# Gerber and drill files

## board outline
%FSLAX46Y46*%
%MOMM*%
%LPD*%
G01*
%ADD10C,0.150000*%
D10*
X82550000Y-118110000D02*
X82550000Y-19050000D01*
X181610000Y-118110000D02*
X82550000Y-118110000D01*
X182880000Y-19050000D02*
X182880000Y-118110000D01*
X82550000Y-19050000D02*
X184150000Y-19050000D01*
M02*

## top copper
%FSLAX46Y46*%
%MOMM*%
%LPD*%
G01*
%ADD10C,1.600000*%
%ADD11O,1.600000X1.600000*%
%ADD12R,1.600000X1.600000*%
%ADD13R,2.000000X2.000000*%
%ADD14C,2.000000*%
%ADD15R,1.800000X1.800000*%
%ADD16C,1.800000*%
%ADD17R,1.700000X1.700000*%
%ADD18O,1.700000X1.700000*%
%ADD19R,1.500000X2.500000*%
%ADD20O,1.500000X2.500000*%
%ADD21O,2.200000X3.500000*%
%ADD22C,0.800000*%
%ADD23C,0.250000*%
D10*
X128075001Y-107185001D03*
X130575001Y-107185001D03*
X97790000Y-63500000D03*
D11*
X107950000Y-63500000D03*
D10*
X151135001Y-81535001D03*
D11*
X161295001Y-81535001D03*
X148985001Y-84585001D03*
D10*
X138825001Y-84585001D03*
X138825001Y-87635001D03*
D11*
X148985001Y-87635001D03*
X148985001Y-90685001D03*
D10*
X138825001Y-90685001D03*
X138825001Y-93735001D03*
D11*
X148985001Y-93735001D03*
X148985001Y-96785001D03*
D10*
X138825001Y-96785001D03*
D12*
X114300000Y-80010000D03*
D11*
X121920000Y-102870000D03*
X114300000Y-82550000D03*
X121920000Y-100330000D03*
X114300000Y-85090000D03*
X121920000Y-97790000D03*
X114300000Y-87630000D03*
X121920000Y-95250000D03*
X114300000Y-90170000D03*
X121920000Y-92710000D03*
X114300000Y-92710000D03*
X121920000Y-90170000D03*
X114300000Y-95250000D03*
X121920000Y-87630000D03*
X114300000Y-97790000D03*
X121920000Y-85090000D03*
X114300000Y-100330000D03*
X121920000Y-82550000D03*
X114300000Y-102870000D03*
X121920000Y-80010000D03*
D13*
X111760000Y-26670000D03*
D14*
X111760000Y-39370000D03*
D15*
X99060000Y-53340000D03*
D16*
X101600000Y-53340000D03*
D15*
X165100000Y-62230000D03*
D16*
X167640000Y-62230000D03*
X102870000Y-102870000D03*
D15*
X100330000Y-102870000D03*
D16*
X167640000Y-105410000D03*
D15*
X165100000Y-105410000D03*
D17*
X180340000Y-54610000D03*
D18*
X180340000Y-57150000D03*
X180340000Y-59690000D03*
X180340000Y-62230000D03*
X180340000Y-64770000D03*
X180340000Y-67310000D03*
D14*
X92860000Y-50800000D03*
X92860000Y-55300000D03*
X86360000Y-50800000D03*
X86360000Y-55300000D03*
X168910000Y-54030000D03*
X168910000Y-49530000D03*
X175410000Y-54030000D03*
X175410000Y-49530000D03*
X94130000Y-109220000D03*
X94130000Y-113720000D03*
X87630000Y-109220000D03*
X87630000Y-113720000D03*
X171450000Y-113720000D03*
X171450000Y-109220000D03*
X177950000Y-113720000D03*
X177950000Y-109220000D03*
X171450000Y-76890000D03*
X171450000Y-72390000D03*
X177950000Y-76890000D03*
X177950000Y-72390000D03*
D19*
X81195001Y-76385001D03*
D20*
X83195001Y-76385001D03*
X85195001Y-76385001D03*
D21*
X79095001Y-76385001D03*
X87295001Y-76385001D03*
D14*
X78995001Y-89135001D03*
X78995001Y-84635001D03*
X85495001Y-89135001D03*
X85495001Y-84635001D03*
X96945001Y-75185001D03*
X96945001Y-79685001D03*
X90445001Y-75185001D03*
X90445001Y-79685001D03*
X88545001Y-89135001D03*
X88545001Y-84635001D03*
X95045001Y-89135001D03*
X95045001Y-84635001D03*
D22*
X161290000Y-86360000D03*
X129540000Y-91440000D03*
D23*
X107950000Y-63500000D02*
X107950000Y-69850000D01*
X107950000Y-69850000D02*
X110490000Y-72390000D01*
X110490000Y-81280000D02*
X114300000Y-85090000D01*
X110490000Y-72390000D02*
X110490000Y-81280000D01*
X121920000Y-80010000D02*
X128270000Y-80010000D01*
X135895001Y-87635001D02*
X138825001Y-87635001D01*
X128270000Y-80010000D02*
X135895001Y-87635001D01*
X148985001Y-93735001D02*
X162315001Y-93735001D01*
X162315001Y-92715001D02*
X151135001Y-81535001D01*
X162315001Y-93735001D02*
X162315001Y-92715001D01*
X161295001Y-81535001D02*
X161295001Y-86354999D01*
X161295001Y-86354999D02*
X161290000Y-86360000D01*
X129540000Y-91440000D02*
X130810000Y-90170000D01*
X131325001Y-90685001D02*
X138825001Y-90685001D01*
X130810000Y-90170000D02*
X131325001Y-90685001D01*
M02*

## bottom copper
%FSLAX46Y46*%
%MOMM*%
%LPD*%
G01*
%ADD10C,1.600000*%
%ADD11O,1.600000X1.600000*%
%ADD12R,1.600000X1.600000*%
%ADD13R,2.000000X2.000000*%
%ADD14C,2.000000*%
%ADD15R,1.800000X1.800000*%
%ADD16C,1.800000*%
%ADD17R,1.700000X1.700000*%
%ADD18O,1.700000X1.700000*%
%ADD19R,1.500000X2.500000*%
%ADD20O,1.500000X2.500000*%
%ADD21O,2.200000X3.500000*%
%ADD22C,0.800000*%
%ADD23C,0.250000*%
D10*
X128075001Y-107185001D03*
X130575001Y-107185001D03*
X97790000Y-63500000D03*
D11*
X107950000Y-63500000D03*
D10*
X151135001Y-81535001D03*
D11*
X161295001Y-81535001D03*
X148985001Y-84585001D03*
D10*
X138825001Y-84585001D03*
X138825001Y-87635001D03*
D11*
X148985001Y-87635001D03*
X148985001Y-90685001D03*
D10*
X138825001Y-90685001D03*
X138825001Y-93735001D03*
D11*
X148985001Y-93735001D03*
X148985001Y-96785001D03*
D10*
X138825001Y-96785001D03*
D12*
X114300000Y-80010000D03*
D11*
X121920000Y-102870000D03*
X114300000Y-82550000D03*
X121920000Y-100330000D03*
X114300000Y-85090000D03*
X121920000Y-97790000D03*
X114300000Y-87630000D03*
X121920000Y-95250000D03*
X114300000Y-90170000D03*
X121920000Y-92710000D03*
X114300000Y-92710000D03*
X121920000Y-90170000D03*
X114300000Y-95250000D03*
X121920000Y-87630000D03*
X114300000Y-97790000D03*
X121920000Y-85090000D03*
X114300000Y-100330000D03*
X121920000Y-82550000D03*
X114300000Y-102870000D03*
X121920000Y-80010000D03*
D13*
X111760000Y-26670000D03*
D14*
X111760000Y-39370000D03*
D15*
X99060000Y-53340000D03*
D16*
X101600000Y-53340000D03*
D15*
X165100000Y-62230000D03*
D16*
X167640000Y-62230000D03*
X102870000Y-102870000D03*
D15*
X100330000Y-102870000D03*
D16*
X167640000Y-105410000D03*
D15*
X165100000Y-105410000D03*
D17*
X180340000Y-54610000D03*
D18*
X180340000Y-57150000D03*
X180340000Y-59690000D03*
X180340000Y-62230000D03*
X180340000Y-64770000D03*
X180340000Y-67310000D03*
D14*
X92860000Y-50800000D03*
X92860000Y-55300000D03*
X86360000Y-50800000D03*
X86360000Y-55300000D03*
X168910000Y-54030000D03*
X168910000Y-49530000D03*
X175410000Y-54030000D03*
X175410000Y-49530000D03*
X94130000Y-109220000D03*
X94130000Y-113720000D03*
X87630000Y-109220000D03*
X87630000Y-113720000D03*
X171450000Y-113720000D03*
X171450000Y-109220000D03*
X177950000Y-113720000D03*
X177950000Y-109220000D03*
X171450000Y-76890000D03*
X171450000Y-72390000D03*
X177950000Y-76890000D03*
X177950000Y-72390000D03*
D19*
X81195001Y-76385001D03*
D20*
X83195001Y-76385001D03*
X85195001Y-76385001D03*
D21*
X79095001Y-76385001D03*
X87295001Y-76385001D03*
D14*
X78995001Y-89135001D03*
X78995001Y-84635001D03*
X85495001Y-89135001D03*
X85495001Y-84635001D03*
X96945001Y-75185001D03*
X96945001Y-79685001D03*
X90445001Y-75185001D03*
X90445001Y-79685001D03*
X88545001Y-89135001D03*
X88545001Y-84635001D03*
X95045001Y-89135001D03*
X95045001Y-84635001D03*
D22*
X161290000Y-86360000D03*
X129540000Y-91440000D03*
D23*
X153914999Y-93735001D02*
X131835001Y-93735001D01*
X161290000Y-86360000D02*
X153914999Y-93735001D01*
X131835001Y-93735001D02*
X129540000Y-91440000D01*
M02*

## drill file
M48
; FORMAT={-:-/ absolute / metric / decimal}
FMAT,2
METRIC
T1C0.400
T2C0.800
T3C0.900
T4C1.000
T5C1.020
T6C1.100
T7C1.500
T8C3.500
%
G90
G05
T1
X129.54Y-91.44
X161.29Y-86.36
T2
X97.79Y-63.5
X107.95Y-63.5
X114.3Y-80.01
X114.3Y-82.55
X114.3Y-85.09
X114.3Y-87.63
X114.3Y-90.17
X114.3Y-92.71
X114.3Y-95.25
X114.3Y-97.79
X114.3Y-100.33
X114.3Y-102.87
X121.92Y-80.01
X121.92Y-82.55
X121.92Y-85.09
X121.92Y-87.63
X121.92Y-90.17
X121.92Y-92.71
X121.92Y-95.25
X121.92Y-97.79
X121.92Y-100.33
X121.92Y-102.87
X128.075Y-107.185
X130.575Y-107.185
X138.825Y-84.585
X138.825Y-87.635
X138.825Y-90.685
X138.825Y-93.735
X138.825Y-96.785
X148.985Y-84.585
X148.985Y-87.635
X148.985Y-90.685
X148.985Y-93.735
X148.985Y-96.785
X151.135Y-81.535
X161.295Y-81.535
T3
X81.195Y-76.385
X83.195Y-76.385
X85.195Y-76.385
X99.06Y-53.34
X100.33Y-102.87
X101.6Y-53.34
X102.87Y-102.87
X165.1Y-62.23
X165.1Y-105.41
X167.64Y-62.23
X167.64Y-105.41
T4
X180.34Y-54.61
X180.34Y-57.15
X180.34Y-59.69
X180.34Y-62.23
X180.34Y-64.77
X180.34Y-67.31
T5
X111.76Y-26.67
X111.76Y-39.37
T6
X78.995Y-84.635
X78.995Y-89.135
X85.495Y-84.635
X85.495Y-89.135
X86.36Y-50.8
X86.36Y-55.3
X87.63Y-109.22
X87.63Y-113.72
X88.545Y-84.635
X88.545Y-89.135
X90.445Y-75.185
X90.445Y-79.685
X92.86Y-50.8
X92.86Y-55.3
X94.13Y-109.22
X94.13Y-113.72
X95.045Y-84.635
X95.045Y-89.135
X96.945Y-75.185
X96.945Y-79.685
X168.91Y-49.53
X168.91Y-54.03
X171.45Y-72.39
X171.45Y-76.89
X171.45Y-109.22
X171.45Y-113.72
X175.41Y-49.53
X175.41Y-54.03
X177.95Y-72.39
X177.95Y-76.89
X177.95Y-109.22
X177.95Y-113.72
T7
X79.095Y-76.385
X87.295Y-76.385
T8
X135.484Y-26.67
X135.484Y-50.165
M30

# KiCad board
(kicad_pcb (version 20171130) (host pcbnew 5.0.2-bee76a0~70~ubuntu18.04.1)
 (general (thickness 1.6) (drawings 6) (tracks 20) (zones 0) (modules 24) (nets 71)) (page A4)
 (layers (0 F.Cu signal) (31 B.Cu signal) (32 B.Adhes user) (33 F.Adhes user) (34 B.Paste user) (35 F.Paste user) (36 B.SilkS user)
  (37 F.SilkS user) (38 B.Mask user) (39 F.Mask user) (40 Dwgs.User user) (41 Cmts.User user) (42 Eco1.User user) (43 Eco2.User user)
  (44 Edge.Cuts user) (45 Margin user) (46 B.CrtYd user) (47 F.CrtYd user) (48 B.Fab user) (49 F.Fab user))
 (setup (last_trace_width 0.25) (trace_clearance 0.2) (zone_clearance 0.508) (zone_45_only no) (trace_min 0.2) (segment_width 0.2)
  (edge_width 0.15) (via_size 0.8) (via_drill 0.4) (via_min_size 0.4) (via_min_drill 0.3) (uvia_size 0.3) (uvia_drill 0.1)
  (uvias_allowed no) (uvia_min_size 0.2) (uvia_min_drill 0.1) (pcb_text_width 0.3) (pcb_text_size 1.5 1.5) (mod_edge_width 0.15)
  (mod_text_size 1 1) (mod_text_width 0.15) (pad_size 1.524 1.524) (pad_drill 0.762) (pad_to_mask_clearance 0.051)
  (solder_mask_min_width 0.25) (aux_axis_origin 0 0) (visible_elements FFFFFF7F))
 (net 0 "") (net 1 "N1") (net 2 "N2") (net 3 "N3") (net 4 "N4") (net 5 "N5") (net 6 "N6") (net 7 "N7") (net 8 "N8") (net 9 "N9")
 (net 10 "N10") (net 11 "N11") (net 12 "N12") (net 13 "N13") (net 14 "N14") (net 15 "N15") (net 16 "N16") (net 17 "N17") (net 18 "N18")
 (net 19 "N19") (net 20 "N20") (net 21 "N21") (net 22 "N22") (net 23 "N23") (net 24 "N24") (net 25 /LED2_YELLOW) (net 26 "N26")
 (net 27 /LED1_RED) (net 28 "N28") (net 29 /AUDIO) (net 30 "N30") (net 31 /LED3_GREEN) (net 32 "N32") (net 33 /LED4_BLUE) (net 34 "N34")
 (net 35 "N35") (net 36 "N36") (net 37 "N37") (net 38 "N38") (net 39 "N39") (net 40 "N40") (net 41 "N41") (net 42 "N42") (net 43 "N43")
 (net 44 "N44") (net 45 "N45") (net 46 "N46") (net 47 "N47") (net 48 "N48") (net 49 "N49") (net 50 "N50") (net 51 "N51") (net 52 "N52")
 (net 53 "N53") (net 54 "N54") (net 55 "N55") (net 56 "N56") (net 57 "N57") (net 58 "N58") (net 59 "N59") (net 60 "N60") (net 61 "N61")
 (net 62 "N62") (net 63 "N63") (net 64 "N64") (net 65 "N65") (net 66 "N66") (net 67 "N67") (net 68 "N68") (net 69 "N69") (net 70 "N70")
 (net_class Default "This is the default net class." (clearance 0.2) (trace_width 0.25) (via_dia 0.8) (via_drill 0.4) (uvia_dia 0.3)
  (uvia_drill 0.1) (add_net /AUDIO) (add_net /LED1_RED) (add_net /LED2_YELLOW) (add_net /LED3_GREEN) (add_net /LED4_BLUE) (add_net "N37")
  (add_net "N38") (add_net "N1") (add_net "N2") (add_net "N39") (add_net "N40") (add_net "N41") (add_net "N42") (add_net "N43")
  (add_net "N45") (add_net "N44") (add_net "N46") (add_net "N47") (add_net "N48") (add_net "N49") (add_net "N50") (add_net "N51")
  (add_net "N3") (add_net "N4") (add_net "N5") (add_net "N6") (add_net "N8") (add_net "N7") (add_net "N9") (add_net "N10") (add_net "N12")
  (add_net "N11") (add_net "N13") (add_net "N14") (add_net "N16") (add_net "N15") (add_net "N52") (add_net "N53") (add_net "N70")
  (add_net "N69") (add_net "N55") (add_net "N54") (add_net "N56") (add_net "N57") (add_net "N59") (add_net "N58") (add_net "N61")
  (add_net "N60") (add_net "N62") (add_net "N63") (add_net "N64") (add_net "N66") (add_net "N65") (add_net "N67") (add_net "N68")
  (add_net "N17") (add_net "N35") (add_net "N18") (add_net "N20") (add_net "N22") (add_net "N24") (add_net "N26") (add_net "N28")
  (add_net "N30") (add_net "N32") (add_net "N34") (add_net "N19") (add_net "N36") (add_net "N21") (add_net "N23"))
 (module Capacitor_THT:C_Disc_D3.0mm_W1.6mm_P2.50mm (layer F.Cu) (at 128.075001 107.185001)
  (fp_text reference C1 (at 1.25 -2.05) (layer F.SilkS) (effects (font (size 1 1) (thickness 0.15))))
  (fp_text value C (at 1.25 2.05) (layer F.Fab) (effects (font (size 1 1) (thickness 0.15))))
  (pad 1 thru_hole circle (at 0 0) (size 1.6 1.6) (drill 0.8) (layers *.Cu *.Mask) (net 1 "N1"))
  (pad 2 thru_hole circle (at 2.5 0) (size 1.6 1.6) (drill 0.8) (layers *.Cu *.Mask) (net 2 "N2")))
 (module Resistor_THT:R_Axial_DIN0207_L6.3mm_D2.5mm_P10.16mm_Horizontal (layer F.Cu) (at 97.79 63.5)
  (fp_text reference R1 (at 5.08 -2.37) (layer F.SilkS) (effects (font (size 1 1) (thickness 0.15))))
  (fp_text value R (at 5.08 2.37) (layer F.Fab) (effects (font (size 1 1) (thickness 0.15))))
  (pad 1 thru_hole circle (at 0 0) (size 1.6 1.6) (drill 0.8) (layers *.Cu *.Mask) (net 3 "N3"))
  (pad 2 thru_hole oval (at 10.16 0) (size 1.6 1.6) (drill 0.8) (layers *.Cu *.Mask) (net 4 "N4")))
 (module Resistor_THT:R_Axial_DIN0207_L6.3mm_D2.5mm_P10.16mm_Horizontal (layer F.Cu) (at 151.135001 81.535001)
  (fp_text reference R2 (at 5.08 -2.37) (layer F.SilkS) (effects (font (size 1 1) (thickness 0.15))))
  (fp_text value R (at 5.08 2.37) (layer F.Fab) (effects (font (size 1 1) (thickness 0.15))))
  (pad 1 thru_hole circle (at 0 0) (size 1.6 1.6) (drill 0.8) (layers *.Cu *.Mask) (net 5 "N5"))
  (pad 2 thru_hole oval (at 10.16 0) (size 1.6 1.6) (drill 0.8) (layers *.Cu *.Mask) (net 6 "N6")))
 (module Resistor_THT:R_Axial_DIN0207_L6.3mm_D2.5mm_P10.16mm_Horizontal (layer F.Cu) (at 138.825001 84.585001)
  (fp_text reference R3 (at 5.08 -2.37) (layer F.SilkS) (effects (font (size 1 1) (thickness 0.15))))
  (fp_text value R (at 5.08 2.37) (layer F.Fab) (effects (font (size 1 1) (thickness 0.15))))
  (pad 2 thru_hole oval (at 10.16 0) (size 1.6 1.6) (drill 0.8) (layers *.Cu *.Mask) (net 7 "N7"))
  (pad 1 thru_hole circle (at 0 0) (size 1.6 1.6) (drill 0.8) (layers *.Cu *.Mask) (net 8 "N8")))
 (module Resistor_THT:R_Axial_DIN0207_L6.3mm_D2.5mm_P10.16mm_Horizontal (layer F.Cu) (at 138.825001 87.635001)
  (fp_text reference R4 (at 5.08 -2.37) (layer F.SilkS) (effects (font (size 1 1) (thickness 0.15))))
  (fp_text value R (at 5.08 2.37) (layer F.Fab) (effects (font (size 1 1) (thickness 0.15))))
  (pad 1 thru_hole circle (at 0 0) (size 1.6 1.6) (drill 0.8) (layers *.Cu *.Mask) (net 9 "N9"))
  (pad 2 thru_hole oval (at 10.16 0) (size 1.6 1.6) (drill 0.8) (layers *.Cu *.Mask) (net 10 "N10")))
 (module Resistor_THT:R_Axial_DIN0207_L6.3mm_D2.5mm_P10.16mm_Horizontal (layer F.Cu) (at 138.825001 90.685001)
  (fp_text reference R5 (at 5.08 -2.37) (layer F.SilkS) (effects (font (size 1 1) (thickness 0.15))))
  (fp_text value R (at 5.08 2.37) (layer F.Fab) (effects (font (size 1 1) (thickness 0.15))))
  (pad 2 thru_hole oval (at 10.16 0) (size 1.6 1.6) (drill 0.8) (layers *.Cu *.Mask) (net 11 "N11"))
  (pad 1 thru_hole circle (at 0 0) (size 1.6 1.6) (drill 0.8) (layers *.Cu *.Mask) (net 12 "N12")))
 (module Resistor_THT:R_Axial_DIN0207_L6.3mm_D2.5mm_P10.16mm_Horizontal (layer F.Cu) (at 138.825001 93.735001)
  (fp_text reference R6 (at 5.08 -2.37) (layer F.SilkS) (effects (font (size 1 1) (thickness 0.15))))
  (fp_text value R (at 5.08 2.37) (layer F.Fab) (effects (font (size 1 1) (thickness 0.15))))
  (pad 1 thru_hole circle (at 0 0) (size 1.6 1.6) (drill 0.8) (layers *.Cu *.Mask) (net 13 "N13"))
  (pad 2 thru_hole oval (at 10.16 0) (size 1.6 1.6) (drill 0.8) (layers *.Cu *.Mask) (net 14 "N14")))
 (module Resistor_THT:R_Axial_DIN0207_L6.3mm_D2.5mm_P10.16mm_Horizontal (layer F.Cu) (at 138.825001 96.785001)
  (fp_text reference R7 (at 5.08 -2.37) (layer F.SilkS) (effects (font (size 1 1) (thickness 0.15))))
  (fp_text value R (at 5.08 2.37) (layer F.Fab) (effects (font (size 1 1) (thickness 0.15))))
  (pad 2 thru_hole oval (at 10.16 0) (size 1.6 1.6) (drill 0.8) (layers *.Cu *.Mask) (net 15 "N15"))
  (pad 1 thru_hole circle (at 0 0) (size 1.6 1.6) (drill 0.8) (layers *.Cu *.Mask) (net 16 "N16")))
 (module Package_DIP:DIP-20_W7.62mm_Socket (layer F.Cu) (at 114.3 80.01)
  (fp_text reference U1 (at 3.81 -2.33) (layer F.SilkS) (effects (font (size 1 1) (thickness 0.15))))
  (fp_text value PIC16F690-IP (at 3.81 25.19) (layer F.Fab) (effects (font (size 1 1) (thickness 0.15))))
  (pad 1 thru_hole rect (at 0 0) (size 1.6 1.6) (drill 0.8) (layers *.Cu *.Mask) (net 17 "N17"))
  (pad 11 thru_hole oval (at 7.62 22.86) (size 1.6 1.6) (drill 0.8) (layers *.Cu *.Mask) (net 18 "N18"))
  (pad 2 thru_hole oval (at 0 2.54) (size 1.6 1.6) (drill 0.8) (layers *.Cu *.Mask) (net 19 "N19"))
  (pad 12 thru_hole oval (at 7.62 20.32) (size 1.6 1.6) (drill 0.8) (layers *.Cu *.Mask) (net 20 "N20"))
  (pad 3 thru_hole oval (at 0 5.08) (size 1.6 1.6) (drill 0.8) (layers *.Cu *.Mask) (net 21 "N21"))
  (pad 13 thru_hole oval (at 7.62 17.78) (size 1.6 1.6) (drill 0.8) (layers *.Cu *.Mask) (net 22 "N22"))
  (pad 4 thru_hole oval (at 0 7.62) (size 1.6 1.6) (drill 0.8) (layers *.Cu *.Mask) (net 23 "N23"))
  (pad 14 thru_hole oval (at 7.62 15.24) (size 1.6 1.6) (drill 0.8) (layers *.Cu *.Mask) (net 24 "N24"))
  (pad 5 thru_hole oval (at 0 10.16) (size 1.6 1.6) (drill 0.8) (layers *.Cu *.Mask) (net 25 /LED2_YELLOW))
  (pad 15 thru_hole oval (at 7.62 12.7) (size 1.6 1.6) (drill 0.8) (layers *.Cu *.Mask) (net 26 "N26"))
  (pad 6 thru_hole oval (at 0 12.7) (size 1.6 1.6) (drill 0.8) (layers *.Cu *.Mask) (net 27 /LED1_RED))
  (pad 16 thru_hole oval (at 7.62 10.16) (size 1.6 1.6) (drill 0.8) (layers *.Cu *.Mask) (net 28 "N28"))
  (pad 7 thru_hole oval (at 0 15.24) (size 1.6 1.6) (drill 0.8) (layers *.Cu *.Mask) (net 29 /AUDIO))
  (pad 17 thru_hole oval (at 7.62 7.62) (size 1.6 1.6) (drill 0.8) (layers *.Cu *.Mask) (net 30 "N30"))
  (pad 8 thru_hole oval (at 0 17.78) (size 1.6 1.6) (drill 0.8) (layers *.Cu *.Mask) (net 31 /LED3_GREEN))
  (pad 18 thru_hole oval (at 7.62 5.08) (size 1.6 1.6) (drill 0.8) (layers *.Cu *.Mask) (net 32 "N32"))
  (pad 9 thru_hole oval (at 0 20.32) (size 1.6 1.6) (drill 0.8) (layers *.Cu *.Mask) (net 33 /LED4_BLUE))
  (pad 19 thru_hole oval (at 7.62 2.54) (size 1.6 1.6) (drill 0.8) (layers *.Cu *.Mask) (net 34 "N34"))
  (pad 10 thru_hole oval (at 0 22.86) (size 1.6 1.6) (drill 0.8) (layers *.Cu *.Mask) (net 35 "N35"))
  (pad 20 thru_hole oval (at 7.62 0) (size 1.6 1.6) (drill 0.8) (layers *.Cu *.Mask) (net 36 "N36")))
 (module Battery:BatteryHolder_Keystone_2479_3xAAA (layer F.Cu) (at 111.76 26.67)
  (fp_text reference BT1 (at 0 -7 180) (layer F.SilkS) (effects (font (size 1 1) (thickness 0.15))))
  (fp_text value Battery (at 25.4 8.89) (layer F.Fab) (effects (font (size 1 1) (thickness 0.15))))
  (pad 1 thru_hole rect (at 0 0) (size 2 2) (drill 1.02) (layers *.Cu *.Mask) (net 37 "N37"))
  (pad 2 thru_hole circle (at 0 12.7) (size 2 2) (drill 1.02) (layers *.Cu *.Mask) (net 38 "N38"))
  (pad "" np_thru_hole circle (at 23.7236 23.495) (size 3.5 3.5) (drill 3.5) (layers *.Cu *.Mask))
  (pad "" np_thru_hole circle (at 23.7236 0) (size 3.5 3.5) (drill 3.5) (layers *.Cu *.Mask)))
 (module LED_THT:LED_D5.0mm (layer F.Cu) (at 99.06 53.34)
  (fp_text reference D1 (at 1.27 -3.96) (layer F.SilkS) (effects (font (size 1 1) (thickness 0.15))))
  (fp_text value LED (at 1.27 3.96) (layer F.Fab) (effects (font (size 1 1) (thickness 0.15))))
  (pad 1 thru_hole rect (at 0 0) (size 1.8 1.8) (drill 0.9) (layers *.Cu *.Mask) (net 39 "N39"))
  (pad 2 thru_hole circle (at 2.54 0) (size 1.8 1.8) (drill 0.9) (layers *.Cu *.Mask) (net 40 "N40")))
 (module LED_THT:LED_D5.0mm (layer F.Cu) (at 165.1 62.23)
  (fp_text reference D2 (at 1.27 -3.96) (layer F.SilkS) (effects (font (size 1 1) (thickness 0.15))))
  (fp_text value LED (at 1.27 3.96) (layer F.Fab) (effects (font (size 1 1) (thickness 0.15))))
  (pad 1 thru_hole rect (at 0 0) (size 1.8 1.8) (drill 0.9) (layers *.Cu *.Mask) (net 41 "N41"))
  (pad 2 thru_hole circle (at 2.54 0) (size 1.8 1.8) (drill 0.9) (layers *.Cu *.Mask) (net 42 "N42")))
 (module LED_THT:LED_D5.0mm (layer F.Cu) (at 100.33 102.87)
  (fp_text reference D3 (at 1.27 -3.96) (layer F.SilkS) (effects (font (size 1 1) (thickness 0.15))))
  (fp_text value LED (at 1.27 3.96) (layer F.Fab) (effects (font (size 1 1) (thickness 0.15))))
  (pad 2 thru_hole circle (at 2.54 0) (size 1.8 1.8) (drill 0.9) (layers *.Cu *.Mask) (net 31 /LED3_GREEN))
  (pad 1 thru_hole rect (at 0 0) (size 1.8 1.8) (drill 0.9) (layers *.Cu *.Mask) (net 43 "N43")))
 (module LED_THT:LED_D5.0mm (layer F.Cu) (at 165.1 105.41)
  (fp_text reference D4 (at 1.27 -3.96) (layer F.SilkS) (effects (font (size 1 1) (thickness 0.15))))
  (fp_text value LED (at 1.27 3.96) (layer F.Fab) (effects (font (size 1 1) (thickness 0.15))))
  (pad 2 thru_hole circle (at 2.54 0) (size 1.8 1.8) (drill 0.9) (layers *.Cu *.Mask) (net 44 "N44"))
  (pad 1 thru_hole rect (at 0 0) (size 1.8 1.8) (drill 0.9) (layers *.Cu *.Mask) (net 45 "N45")))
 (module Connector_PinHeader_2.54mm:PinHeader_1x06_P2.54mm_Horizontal (layer F.Cu) (at 180.34 54.61)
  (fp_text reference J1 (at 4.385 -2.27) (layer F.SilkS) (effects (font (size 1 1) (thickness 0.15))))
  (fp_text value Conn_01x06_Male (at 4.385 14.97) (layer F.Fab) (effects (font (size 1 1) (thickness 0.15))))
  (pad 1 thru_hole rect (at 0 0) (size 1.7 1.7) (drill 1) (layers *.Cu *.Mask) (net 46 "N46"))
  (pad 2 thru_hole oval (at 0 2.54) (size 1.7 1.7) (drill 1) (layers *.Cu *.Mask) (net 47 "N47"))
  (pad 3 thru_hole oval (at 0 5.08) (size 1.7 1.7) (drill 1) (layers *.Cu *.Mask) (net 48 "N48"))
  (pad 4 thru_hole oval (at 0 7.62) (size 1.7 1.7) (drill 1) (layers *.Cu *.Mask) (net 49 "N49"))
  (pad 5 thru_hole oval (at 0 10.16) (size 1.7 1.7) (drill 1) (layers *.Cu *.Mask) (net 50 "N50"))
  (pad 6 thru_hole oval (at 0 12.7) (size 1.7 1.7) (drill 1) (layers *.Cu *.Mask) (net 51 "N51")))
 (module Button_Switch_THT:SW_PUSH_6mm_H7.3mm (layer F.Cu) (at 86.36 50.8)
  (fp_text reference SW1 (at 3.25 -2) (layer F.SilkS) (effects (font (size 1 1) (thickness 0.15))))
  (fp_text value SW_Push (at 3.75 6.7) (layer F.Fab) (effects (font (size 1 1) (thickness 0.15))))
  (pad 1 thru_hole circle (at 6.5 0 90) (size 2 2) (drill 1.1) (layers *.Cu *.Mask) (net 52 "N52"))
  (pad 2 thru_hole circle (at 6.5 4.5 90) (size 2 2) (drill 1.1) (layers *.Cu *.Mask) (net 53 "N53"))
  (pad 1 thru_hole circle (at 0 0 90) (size 2 2) (drill 1.1) (layers *.Cu *.Mask) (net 52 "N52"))
  (pad 2 thru_hole circle (at 0 4.5 90) (size 2 2) (drill 1.1) (layers *.Cu *.Mask) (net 53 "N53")))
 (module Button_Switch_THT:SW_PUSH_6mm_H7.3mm (layer F.Cu) (at 168.91 49.53)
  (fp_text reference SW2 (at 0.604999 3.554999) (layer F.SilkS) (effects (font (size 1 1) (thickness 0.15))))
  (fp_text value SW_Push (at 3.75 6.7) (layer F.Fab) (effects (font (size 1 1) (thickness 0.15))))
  (pad 2 thru_hole circle (at 0 4.5 90) (size 2 2) (drill 1.1) (layers *.Cu *.Mask) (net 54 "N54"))
  (pad 1 thru_hole circle (at 0 0 90) (size 2 2) (drill 1.1) (layers *.Cu *.Mask) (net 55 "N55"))
  (pad 2 thru_hole circle (at 6.5 4.5 90) (size 2 2) (drill 1.1) (layers *.Cu *.Mask) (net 54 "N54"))
  (pad 1 thru_hole circle (at 6.5 0 90) (size 2 2) (drill 1.1) (layers *.Cu *.Mask) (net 55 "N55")))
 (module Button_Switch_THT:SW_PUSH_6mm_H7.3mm (layer F.Cu) (at 87.63 109.22)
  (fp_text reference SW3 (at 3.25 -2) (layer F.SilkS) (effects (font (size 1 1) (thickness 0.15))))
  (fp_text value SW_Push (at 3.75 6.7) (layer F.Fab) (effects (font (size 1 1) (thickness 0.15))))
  (pad 1 thru_hole circle (at 6.5 0 90) (size 2 2) (drill 1.1) (layers *.Cu *.Mask) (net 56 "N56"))
  (pad 2 thru_hole circle (at 6.5 4.5 90) (size 2 2) (drill 1.1) (layers *.Cu *.Mask) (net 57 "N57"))
  (pad 1 thru_hole circle (at 0 0 90) (size 2 2) (drill 1.1) (layers *.Cu *.Mask) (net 56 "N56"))
  (pad 2 thru_hole circle (at 0 4.5 90) (size 2 2) (drill 1.1) (layers *.Cu *.Mask) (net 57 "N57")))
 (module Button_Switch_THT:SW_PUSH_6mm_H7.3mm (layer F.Cu) (at 171.45 109.22)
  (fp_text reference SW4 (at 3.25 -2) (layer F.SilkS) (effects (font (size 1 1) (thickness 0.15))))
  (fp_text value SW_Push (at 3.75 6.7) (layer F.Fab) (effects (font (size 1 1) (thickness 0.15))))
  (pad 2 thru_hole circle (at 0 4.5 90) (size 2 2) (drill 1.1) (layers *.Cu *.Mask) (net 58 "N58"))
  (pad 1 thru_hole circle (at 0 0 90) (size 2 2) (drill 1.1) (layers *.Cu *.Mask) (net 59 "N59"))
  (pad 2 thru_hole circle (at 6.5 4.5 90) (size 2 2) (drill 1.1) (layers *.Cu *.Mask) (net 58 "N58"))
  (pad 1 thru_hole circle (at 6.5 0 90) (size 2 2) (drill 1.1) (layers *.Cu *.Mask) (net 59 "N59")))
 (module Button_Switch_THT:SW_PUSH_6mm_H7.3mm (layer F.Cu) (at 171.45 72.39)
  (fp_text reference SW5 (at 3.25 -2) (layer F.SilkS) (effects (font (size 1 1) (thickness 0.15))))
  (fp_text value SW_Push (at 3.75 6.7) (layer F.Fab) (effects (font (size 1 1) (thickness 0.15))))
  (pad 2 thru_hole circle (at 0 4.5 90) (size 2 2) (drill 1.1) (layers *.Cu *.Mask) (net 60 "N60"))
  (pad 1 thru_hole circle (at 0 0 90) (size 2 2) (drill 1.1) (layers *.Cu *.Mask) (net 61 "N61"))
  (pad 2 thru_hole circle (at 6.5 4.5 90) (size 2 2) (drill 1.1) (layers *.Cu *.Mask) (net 60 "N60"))
  (pad 1 thru_hole circle (at 6.5 0 90) (size 2 2) (drill 1.1) (layers *.Cu *.Mask) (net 61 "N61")))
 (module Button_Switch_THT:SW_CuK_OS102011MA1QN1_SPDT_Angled (layer F.Cu) (at 81.195001 76.385001)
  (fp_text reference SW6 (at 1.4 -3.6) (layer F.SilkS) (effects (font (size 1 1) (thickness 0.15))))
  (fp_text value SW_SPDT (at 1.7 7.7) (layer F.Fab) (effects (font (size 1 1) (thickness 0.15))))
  (pad 1 thru_hole rect (at 0 0) (size 1.5 2.5) (drill 0.9) (layers *.Cu *.Mask) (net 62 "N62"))
  (pad 2 thru_hole oval (at 2 0) (size 1.5 2.5) (drill 0.9) (layers *.Cu *.Mask) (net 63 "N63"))
  (pad 3 thru_hole oval (at 4 0) (size 1.5 2.5) (drill 0.9) (layers *.Cu *.Mask) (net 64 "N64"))
  (pad "" thru_hole oval (at -2.1 0) (size 2.2 3.5) (drill 1.5) (layers *.Cu *.Mask))
  (pad "" thru_hole oval (at 6.1 0) (size 2.2 3.5) (drill 1.5) (layers *.Cu *.Mask)))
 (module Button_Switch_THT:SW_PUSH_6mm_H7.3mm (layer F.Cu) (at 78.995001 84.635001)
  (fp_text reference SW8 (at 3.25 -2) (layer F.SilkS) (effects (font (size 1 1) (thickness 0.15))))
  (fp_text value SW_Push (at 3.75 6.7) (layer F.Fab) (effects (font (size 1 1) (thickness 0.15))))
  (pad 2 thru_hole circle (at 0 4.5 90) (size 2 2) (drill 1.1) (layers *.Cu *.Mask) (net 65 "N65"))
  (pad 1 thru_hole circle (at 0 0 90) (size 2 2) (drill 1.1) (layers *.Cu *.Mask) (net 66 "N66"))
  (pad 2 thru_hole circle (at 6.5 4.5 90) (size 2 2) (drill 1.1) (layers *.Cu *.Mask) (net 65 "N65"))
  (pad 1 thru_hole circle (at 6.5 0 90) (size 2 2) (drill 1.1) (layers *.Cu *.Mask) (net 66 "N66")))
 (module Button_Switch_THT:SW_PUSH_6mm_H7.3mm (layer F.Cu) (at 90.445001 75.185001)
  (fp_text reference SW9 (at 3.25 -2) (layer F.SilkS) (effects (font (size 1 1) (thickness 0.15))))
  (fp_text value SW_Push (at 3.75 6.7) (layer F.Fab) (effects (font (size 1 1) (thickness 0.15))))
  (pad 1 thru_hole circle (at 6.5 0 90) (size 2 2) (drill 1.1) (layers *.Cu *.Mask) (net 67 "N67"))
  (pad 2 thru_hole circle (at 6.5 4.5 90) (size 2 2) (drill 1.1) (layers *.Cu *.Mask) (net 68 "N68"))
  (pad 1 thru_hole circle (at 0 0 90) (size 2 2) (drill 1.1) (layers *.Cu *.Mask) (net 67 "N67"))
  (pad 2 thru_hole circle (at 0 4.5 90) (size 2 2) (drill 1.1) (layers *.Cu *.Mask) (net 68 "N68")))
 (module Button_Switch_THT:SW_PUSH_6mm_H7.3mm (layer F.Cu) (at 88.545001 84.635001)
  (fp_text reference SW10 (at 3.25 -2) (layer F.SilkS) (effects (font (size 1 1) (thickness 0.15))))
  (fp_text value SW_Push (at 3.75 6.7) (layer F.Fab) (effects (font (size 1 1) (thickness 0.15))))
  (pad 2 thru_hole circle (at 0 4.5 90) (size 2 2) (drill 1.1) (layers *.Cu *.Mask) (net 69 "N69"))
  (pad 1 thru_hole circle (at 0 0 90) (size 2 2) (drill 1.1) (layers *.Cu *.Mask) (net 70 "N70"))
  (pad 2 thru_hole circle (at 6.5 4.5 90) (size 2 2) (drill 1.1) (layers *.Cu *.Mask) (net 69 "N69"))
  (pad 1 thru_hole circle (at 6.5 0 90) (size 2 2) (drill 1.1) (layers *.Cu *.Mask) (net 70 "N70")))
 (gr_line (start 82.55 118.11) (end 82.55 19.05) (layer Edge.Cuts) (width 0.15))
 (gr_line (start 181.61 118.11) (end 82.55 118.11) (layer Edge.Cuts) (width 0.15))
 (gr_line (start 182.88 19.05) (end 182.88 118.11) (layer Edge.Cuts) (width 0.15))
 (gr_line (start 82.55 19.05) (end 184.15 19.05) (layer Edge.Cuts) (width 0.15))
 (segment (start 107.95 63.5) (end 107.95 69.85) (width 0.25) (layer F.Cu) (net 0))
 (segment (start 107.95 69.85) (end 110.49 72.39) (width 0.25) (layer F.Cu) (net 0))
 (segment (start 110.49 81.28) (end 114.3 85.09) (width 0.25) (layer F.Cu) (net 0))
 (segment (start 110.49 72.39) (end 110.49 81.28) (width 0.25) (layer F.Cu) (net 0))
 (segment (start 121.92 80.01) (end 128.27 80.01) (width 0.25) (layer F.Cu) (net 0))
 (segment (start 135.895001 87.635001) (end 138.825001 87.635001) (width 0.25) (layer F.Cu) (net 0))
 (segment (start 128.27 80.01) (end 135.895001 87.635001) (width 0.25) (layer F.Cu) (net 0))
 (segment (start 148.985001 93.735001) (end 162.315001 93.735001) (width 0.25) (layer F.Cu) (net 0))
 (segment (start 162.315001 92.715001) (end 151.135001 81.535001) (width 0.25) (layer F.Cu) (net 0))
 (segment (start 162.315001 93.735001) (end 162.315001 92.715001) (width 0.25) (layer F.Cu) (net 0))
 (segment (start 161.295001 81.535001) (end 161.295001 86.354999) (width 0.25) (layer F.Cu) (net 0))
 (via (at 161.29 86.36) (size 0.8) (drill 0.4) (layers F.Cu B.Cu) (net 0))
 (segment (start 161.295001 86.354999) (end 161.29 86.36) (width 0.25) (layer F.Cu) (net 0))
 (segment (start 153.914999 93.735001) (end 131.835001 93.735001) (width 0.25) (layer B.Cu) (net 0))
 (segment (start 161.29 86.36) (end 153.914999 93.735001) (width 0.25) (layer B.Cu) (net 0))
 (via (at 129.54 91.44) (size 0.8) (drill 0.4) (layers F.Cu B.Cu) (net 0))
 (segment (start 131.835001 93.735001) (end 129.54 91.44) (width 0.25) (layer B.Cu) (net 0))
 (segment (start 129.54 91.44) (end 130.81 90.17) (width 0.25) (layer F.Cu) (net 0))
 (segment (start 131.325001 90.685001) (end 138.825001 90.685001) (width 0.25) (layer F.Cu) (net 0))
 (segment (start 130.81 90.17) (end 131.325001 90.685001) (width 0.25) (layer F.Cu) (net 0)))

